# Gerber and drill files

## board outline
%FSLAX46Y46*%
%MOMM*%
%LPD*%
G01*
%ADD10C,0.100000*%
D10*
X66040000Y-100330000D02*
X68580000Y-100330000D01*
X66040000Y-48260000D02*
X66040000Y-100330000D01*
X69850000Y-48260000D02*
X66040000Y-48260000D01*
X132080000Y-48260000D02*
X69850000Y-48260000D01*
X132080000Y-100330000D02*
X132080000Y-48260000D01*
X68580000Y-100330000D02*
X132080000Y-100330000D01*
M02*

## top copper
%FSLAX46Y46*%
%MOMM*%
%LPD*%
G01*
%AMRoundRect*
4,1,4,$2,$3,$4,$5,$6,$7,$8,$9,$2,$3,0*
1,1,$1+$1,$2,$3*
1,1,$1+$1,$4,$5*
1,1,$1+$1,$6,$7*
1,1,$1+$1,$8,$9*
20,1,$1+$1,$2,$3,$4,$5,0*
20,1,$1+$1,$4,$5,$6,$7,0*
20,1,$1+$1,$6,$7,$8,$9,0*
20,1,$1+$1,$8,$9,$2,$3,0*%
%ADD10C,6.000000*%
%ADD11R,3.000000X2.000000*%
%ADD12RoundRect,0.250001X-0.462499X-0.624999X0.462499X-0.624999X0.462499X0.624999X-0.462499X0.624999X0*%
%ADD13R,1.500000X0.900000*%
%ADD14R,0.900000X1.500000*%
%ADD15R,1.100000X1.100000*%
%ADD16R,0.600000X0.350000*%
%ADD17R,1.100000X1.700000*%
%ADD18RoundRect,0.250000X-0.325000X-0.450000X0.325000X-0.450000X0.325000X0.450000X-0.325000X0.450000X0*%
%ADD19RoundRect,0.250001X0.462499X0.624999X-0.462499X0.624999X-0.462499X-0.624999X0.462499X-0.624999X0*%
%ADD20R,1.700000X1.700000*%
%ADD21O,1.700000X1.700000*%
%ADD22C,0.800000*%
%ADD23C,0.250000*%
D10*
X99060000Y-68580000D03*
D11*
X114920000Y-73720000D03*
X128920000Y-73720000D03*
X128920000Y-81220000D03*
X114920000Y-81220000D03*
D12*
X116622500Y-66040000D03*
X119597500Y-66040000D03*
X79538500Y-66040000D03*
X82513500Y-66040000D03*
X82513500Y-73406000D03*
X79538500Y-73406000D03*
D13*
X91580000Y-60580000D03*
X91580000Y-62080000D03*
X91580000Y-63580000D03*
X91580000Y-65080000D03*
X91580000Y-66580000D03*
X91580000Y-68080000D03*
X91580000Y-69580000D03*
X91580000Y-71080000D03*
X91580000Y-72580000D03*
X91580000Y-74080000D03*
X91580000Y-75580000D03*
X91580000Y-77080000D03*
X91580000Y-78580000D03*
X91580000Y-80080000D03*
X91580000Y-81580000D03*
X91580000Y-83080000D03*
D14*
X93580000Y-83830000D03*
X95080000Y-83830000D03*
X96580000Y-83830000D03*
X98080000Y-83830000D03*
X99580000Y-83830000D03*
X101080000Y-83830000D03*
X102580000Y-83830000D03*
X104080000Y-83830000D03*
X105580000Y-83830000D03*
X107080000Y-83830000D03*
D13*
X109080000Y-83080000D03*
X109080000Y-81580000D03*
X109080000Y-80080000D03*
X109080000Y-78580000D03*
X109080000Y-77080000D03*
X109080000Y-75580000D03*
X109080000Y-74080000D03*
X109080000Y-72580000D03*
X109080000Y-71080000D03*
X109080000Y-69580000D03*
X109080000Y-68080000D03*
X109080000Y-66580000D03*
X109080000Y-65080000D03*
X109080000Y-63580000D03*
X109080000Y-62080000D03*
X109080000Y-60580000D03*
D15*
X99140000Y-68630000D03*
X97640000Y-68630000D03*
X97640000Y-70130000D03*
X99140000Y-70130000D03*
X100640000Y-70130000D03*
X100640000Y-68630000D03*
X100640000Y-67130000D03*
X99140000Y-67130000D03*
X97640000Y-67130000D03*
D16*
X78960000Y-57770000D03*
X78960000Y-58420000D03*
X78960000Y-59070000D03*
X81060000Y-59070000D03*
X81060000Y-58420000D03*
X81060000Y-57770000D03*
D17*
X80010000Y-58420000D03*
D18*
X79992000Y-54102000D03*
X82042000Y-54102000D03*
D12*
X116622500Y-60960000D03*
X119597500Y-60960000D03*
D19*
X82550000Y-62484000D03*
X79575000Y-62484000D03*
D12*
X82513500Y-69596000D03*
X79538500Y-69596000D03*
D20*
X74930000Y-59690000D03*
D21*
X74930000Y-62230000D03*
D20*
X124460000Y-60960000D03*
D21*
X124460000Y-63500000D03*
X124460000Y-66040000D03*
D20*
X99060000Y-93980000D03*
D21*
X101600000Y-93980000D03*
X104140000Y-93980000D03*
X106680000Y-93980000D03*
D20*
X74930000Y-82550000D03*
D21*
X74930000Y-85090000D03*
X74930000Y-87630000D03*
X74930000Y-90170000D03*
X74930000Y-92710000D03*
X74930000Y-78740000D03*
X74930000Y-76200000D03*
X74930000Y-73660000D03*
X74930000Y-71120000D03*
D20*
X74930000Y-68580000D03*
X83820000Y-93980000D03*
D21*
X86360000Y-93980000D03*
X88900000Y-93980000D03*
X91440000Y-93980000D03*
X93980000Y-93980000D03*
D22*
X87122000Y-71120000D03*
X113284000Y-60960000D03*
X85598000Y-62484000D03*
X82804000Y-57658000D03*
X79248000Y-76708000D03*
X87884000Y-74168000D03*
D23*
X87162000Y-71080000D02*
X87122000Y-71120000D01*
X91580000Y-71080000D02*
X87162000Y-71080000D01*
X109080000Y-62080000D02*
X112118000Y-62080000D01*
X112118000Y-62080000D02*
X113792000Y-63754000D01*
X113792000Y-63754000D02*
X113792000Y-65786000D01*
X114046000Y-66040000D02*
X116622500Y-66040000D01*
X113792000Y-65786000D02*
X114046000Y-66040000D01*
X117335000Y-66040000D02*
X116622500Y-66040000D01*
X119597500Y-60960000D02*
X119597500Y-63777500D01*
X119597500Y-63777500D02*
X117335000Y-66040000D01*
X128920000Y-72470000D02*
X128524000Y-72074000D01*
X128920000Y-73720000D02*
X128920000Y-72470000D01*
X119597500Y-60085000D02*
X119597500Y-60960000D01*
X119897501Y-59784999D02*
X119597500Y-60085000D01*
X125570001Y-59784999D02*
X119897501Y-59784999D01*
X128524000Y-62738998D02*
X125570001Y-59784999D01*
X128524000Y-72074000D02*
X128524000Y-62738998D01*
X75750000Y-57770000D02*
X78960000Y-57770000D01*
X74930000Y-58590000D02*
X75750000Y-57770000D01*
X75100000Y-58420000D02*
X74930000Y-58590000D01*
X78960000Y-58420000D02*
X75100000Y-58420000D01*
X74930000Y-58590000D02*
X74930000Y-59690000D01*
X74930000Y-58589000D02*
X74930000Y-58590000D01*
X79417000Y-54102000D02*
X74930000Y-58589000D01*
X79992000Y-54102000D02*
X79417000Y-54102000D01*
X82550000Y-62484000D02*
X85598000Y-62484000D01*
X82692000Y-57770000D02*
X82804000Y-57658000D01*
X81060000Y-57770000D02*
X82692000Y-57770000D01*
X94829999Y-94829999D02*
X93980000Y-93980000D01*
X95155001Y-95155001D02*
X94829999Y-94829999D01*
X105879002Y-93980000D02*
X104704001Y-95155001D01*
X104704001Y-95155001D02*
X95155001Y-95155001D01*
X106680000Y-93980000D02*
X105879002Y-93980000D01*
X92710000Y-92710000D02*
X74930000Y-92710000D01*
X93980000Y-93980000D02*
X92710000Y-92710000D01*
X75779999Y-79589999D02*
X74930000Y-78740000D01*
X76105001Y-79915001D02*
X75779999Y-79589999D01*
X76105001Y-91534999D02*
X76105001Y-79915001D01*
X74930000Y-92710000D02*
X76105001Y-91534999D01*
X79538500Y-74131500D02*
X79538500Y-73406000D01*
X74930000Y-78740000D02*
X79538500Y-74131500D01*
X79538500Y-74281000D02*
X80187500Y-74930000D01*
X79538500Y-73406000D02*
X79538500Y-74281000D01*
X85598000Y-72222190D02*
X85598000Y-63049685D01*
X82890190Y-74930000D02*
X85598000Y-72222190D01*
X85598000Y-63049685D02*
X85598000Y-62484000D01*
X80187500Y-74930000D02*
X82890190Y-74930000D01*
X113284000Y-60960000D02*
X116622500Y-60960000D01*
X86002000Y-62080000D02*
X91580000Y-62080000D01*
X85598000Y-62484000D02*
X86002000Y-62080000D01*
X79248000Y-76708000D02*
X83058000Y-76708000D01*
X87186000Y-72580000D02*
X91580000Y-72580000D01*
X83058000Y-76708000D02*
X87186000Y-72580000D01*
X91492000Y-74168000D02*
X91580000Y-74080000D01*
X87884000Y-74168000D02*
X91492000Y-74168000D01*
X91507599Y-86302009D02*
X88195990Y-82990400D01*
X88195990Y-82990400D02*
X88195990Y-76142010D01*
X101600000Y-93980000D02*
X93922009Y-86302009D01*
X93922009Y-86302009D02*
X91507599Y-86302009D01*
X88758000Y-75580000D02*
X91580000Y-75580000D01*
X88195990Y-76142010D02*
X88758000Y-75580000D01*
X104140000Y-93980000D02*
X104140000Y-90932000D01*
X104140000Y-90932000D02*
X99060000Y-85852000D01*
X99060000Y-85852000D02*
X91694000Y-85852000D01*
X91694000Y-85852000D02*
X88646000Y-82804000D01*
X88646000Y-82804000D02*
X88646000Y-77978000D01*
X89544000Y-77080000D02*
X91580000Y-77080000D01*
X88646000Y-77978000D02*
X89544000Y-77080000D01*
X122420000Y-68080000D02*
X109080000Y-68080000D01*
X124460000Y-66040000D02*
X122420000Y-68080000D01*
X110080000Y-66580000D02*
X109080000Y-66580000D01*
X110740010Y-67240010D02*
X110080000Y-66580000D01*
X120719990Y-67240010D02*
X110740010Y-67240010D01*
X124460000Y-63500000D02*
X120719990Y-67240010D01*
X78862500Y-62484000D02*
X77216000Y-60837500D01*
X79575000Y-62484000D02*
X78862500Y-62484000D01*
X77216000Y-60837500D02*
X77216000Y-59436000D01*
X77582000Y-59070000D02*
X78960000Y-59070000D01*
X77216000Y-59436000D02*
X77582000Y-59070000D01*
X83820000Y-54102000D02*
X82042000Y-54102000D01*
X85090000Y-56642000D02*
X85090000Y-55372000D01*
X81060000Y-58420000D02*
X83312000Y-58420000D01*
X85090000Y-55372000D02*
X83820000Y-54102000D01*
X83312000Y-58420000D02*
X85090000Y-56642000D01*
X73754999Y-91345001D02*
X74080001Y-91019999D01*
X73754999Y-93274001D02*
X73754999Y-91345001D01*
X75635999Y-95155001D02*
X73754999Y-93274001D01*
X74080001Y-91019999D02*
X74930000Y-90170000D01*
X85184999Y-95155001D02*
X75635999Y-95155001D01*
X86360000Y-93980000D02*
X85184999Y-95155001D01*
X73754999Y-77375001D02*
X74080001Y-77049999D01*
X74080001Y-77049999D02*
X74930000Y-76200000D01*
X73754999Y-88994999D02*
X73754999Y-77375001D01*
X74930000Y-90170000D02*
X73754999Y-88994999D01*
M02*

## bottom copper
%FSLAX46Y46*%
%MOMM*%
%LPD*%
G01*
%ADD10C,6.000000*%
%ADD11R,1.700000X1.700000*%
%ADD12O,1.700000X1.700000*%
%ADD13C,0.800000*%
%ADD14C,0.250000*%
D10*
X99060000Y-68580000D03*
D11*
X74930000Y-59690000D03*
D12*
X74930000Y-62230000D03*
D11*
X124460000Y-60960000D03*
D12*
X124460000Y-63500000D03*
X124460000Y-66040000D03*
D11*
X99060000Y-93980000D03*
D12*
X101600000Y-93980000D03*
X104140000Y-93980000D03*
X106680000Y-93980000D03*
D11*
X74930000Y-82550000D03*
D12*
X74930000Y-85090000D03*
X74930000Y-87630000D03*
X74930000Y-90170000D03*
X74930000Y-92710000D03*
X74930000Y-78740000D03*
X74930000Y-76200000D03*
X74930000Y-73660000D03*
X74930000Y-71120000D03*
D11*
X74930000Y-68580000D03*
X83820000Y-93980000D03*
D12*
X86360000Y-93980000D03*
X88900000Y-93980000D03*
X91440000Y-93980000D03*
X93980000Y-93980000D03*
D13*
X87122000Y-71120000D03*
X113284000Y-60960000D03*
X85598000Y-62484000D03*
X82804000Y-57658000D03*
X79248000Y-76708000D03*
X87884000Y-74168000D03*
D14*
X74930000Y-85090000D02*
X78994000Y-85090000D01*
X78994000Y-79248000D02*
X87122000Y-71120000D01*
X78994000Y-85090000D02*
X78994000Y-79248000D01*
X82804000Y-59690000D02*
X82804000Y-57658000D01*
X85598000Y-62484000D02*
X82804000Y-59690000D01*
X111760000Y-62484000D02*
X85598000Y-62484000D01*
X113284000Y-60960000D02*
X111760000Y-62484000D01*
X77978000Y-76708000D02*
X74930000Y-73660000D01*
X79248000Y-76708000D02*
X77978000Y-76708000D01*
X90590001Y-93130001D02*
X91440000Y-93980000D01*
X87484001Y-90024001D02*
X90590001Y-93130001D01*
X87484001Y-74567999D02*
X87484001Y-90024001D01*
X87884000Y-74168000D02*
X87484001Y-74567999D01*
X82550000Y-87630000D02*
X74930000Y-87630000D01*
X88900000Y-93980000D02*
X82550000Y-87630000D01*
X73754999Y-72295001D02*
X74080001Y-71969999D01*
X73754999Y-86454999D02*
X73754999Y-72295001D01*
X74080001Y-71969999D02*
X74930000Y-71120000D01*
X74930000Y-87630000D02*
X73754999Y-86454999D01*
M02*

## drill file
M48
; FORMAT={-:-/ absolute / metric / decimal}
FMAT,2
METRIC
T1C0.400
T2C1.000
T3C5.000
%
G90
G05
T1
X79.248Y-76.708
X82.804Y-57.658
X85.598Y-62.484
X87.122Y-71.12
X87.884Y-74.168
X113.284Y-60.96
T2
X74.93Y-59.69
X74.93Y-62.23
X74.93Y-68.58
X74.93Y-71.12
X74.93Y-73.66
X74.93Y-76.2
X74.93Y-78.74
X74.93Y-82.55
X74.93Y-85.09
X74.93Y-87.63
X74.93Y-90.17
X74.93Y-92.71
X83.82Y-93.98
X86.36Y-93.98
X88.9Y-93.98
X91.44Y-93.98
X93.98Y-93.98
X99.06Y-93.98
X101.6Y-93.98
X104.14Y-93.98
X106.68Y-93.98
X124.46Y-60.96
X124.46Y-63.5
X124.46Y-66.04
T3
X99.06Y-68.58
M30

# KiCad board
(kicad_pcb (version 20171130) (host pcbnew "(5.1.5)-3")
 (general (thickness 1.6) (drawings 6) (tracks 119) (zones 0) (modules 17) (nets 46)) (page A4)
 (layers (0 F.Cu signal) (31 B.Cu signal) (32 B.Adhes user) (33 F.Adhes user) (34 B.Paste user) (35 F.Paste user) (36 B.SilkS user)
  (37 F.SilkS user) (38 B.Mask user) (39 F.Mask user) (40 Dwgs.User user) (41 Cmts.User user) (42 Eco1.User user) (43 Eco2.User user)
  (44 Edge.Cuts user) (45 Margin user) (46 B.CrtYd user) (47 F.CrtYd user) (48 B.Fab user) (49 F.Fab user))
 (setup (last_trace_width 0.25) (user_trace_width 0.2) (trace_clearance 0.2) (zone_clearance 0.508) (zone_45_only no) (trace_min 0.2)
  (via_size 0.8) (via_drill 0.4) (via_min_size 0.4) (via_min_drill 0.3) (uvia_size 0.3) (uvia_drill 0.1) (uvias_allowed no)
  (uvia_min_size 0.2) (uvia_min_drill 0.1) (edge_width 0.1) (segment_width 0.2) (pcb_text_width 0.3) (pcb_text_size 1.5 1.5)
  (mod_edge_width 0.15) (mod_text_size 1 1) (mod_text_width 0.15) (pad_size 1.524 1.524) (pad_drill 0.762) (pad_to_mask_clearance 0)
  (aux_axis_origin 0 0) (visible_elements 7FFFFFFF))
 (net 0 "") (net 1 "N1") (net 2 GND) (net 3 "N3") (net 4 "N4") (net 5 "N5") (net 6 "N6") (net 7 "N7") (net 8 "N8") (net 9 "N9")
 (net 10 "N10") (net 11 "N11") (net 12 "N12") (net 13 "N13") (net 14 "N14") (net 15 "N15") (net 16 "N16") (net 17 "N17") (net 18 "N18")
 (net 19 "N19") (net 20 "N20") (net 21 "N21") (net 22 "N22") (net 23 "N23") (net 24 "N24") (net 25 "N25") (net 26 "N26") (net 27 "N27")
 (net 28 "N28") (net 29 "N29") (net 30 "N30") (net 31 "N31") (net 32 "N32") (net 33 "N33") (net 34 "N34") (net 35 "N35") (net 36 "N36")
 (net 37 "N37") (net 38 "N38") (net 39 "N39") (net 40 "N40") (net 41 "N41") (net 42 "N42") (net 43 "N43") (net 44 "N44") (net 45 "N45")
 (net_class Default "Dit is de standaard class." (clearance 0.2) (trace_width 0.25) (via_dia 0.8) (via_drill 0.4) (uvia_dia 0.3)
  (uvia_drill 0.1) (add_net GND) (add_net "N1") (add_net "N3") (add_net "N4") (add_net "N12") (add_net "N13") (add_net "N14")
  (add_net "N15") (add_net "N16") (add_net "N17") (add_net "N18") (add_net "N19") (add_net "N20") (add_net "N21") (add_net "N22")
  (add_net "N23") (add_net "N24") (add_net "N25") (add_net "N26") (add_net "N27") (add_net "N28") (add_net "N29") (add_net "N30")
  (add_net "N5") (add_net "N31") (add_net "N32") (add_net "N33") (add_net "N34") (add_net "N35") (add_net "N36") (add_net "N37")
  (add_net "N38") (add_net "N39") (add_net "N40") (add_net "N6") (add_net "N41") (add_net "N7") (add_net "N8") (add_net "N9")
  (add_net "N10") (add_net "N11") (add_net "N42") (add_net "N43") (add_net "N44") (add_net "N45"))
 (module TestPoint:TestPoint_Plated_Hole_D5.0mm (layer F.Cu) (at 99.06 68.58)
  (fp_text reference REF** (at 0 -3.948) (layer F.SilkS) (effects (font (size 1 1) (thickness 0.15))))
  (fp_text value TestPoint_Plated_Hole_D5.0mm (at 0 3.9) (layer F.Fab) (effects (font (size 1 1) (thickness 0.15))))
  (pad 1 thru_hole circle (at 0 0) (size 6 6) (drill 5) (layers *.Cu *.Mask)))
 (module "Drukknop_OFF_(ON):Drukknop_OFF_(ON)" (layer F.Cu) (at 121.92 77.47)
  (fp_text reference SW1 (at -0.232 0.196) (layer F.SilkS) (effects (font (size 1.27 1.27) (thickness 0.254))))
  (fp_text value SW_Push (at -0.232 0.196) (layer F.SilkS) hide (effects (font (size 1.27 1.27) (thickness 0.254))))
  (pad 4 smd rect (at -7 -3.75 90) (size 2 3) (layers F.Cu F.Paste F.Mask))
  (pad 3 smd rect (at 7 -3.75 90) (size 2 3) (layers F.Cu F.Paste F.Mask) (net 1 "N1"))
  (pad 2 smd rect (at 7 3.75 90) (size 2 3) (layers F.Cu F.Paste F.Mask))
  (pad 1 smd rect (at -7 3.75 90) (size 2 3) (layers F.Cu F.Paste F.Mask) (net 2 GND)))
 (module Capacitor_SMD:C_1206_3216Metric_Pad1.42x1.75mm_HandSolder (layer F.Cu) (at 118.11 66.04)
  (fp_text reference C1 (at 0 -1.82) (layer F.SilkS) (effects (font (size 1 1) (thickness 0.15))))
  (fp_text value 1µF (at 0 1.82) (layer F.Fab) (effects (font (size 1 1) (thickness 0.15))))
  (pad 1 smd roundrect (at -1.4875 0) (size 1.425 1.75) (layers F.Cu F.Paste F.Mask) (roundrect_rratio 0.175439) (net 1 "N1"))
  (pad 2 smd roundrect (at 1.4875 0) (size 1.425 1.75) (layers F.Cu F.Paste F.Mask) (roundrect_rratio 0.175439) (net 2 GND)))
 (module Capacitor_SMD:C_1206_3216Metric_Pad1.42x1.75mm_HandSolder (layer F.Cu) (at 81.026 66.04)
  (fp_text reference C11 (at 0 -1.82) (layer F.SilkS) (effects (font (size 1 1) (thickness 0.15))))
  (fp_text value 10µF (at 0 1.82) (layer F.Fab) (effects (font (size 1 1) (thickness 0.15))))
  (pad 1 smd roundrect (at -1.4875 0) (size 1.425 1.75) (layers F.Cu F.Paste F.Mask) (roundrect_rratio 0.175439) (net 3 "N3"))
  (pad 2 smd roundrect (at 1.4875 0) (size 1.425 1.75) (layers F.Cu F.Paste F.Mask) (roundrect_rratio 0.175439) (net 2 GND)))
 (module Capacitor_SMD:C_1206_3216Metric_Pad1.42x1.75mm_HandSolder (layer F.Cu) (at 81.026 73.406)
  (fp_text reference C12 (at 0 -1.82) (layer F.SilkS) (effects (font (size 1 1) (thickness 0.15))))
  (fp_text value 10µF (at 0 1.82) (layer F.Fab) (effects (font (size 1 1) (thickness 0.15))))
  (pad 2 smd roundrect (at 1.4875 0) (size 1.425 1.75) (layers F.Cu F.Paste F.Mask) (roundrect_rratio 0.175439) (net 2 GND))
  (pad 1 smd roundrect (at -1.4875 0) (size 1.425 1.75) (layers F.Cu F.Paste F.Mask) (roundrect_rratio 0.175439) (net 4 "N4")))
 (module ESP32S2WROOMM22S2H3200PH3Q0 (layer F.Cu) (at 100.33 68.58)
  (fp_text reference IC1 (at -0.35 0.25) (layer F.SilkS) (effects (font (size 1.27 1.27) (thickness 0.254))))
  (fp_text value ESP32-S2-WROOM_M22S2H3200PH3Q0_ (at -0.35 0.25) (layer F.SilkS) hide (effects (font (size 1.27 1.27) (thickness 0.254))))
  (pad 1 smd rect (at -8.75 -8 90) (size 0.9 1.5) (layers F.Cu F.Paste F.Mask) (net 2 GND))
  (pad 2 smd rect (at -8.75 -6.5 90) (size 0.9 1.5) (layers F.Cu F.Paste F.Mask) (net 4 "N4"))
  (pad 3 smd rect (at -8.75 -5 90) (size 0.9 1.5) (layers F.Cu F.Paste F.Mask) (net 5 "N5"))
  (pad 4 smd rect (at -8.75 -3.5 90) (size 0.9 1.5) (layers F.Cu F.Paste F.Mask) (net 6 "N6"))
  (pad 5 smd rect (at -8.75 -2 90) (size 0.9 1.5) (layers F.Cu F.Paste F.Mask) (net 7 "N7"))
  (pad 6 smd rect (at -8.75 -0.5 90) (size 0.9 1.5) (layers F.Cu F.Paste F.Mask) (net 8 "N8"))
  (pad 7 smd rect (at -8.75 1 90) (size 0.9 1.5) (layers F.Cu F.Paste F.Mask) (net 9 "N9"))
  (pad 8 smd rect (at -8.75 2.5 90) (size 0.9 1.5) (layers F.Cu F.Paste F.Mask) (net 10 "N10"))
  (pad 9 smd rect (at -8.75 4 90) (size 0.9 1.5) (layers F.Cu F.Paste F.Mask) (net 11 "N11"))
  (pad 10 smd rect (at -8.75 5.5 90) (size 0.9 1.5) (layers F.Cu F.Paste F.Mask) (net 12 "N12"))
  (pad 11 smd rect (at -8.75 7 90) (size 0.9 1.5) (layers F.Cu F.Paste F.Mask) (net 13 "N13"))
  (pad 12 smd rect (at -8.75 8.5 90) (size 0.9 1.5) (layers F.Cu F.Paste F.Mask) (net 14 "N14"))
  (pad 13 smd rect (at -8.75 10 90) (size 0.9 1.5) (layers F.Cu F.Paste F.Mask) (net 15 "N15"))
  (pad 14 smd rect (at -8.75 11.5 90) (size 0.9 1.5) (layers F.Cu F.Paste F.Mask) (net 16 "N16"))
  (pad 15 smd rect (at -8.75 13 90) (size 0.9 1.5) (layers F.Cu F.Paste F.Mask) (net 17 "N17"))
  (pad 16 smd rect (at -8.75 14.5 90) (size 0.9 1.5) (layers F.Cu F.Paste F.Mask) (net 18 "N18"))
  (pad 17 smd rect (at -6.75 15.25) (size 0.9 1.5) (layers F.Cu F.Paste F.Mask) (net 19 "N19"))
  (pad 18 smd rect (at -5.25 15.25) (size 0.9 1.5) (layers F.Cu F.Paste F.Mask) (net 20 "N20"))
  (pad 19 smd rect (at -3.75 15.25) (size 0.9 1.5) (layers F.Cu F.Paste F.Mask) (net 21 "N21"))
  (pad 20 smd rect (at -2.25 15.25) (size 0.9 1.5) (layers F.Cu F.Paste F.Mask) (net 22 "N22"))
  (pad 21 smd rect (at -0.75 15.25) (size 0.9 1.5) (layers F.Cu F.Paste F.Mask) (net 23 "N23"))
  (pad 22 smd rect (at 0.75 15.25) (size 0.9 1.5) (layers F.Cu F.Paste F.Mask) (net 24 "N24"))
  (pad 23 smd rect (at 2.25 15.25) (size 0.9 1.5) (layers F.Cu F.Paste F.Mask) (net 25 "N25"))
  (pad 24 smd rect (at 3.75 15.25) (size 0.9 1.5) (layers F.Cu F.Paste F.Mask) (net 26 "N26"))
  (pad 25 smd rect (at 5.25 15.25) (size 0.9 1.5) (layers F.Cu F.Paste F.Mask) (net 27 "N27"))
  (pad 26 smd rect (at 6.75 15.25) (size 0.9 1.5) (layers F.Cu F.Paste F.Mask) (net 2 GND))
  (pad 27 smd rect (at 8.75 14.5 90) (size 0.9 1.5) (layers F.Cu F.Paste F.Mask) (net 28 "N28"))
  (pad 28 smd rect (at 8.75 13 90) (size 0.9 1.5) (layers F.Cu F.Paste F.Mask) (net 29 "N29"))
  (pad 29 smd rect (at 8.75 11.5 90) (size 0.9 1.5) (layers F.Cu F.Paste F.Mask) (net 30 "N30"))
  (pad 30 smd rect (at 8.75 10 90) (size 0.9 1.5) (layers F.Cu F.Paste F.Mask) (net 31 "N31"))
  (pad 31 smd rect (at 8.75 8.5 90) (size 0.9 1.5) (layers F.Cu F.Paste F.Mask) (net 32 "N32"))
  (pad 32 smd rect (at 8.75 7 90) (size 0.9 1.5) (layers F.Cu F.Paste F.Mask) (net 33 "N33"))
  (pad 33 smd rect (at 8.75 5.5 90) (size 0.9 1.5) (layers F.Cu F.Paste F.Mask) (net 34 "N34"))
  (pad 34 smd rect (at 8.75 4 90) (size 0.9 1.5) (layers F.Cu F.Paste F.Mask) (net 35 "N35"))
  (pad 35 smd rect (at 8.75 2.5 90) (size 0.9 1.5) (layers F.Cu F.Paste F.Mask) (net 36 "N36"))
  (pad 36 smd rect (at 8.75 1 90) (size 0.9 1.5) (layers F.Cu F.Paste F.Mask) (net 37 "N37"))
  (pad 37 smd rect (at 8.75 -0.5 90) (size 0.9 1.5) (layers F.Cu F.Paste F.Mask) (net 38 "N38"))
  (pad 38 smd rect (at 8.75 -2 90) (size 0.9 1.5) (layers F.Cu F.Paste F.Mask) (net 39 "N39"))
  (pad 39 smd rect (at 8.75 -3.5 90) (size 0.9 1.5) (layers F.Cu F.Paste F.Mask) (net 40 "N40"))
  (pad 40 smd rect (at 8.75 -5 90) (size 0.9 1.5) (layers F.Cu F.Paste F.Mask) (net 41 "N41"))
  (pad 41 smd rect (at 8.75 -6.5 90) (size 0.9 1.5) (layers F.Cu F.Paste F.Mask) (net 1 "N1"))
  (pad 42 smd rect (at 8.75 -8 90) (size 0.9 1.5) (layers F.Cu F.Paste F.Mask) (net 2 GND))
  (pad 43 smd rect (at -1.19 0.05) (size 1.1 1.1) (layers F.Cu F.Paste F.Mask) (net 2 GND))
  (pad 44 smd rect (at -2.69 0.05) (size 1.1 1.1) (layers F.Cu F.Paste F.Mask) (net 2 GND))
  (pad 45 smd rect (at -2.69 1.55) (size 1.1 1.1) (layers F.Cu F.Paste F.Mask) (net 2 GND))
  (pad 46 smd rect (at -1.19 1.55) (size 1.1 1.1) (layers F.Cu F.Paste F.Mask) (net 2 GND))
  (pad 47 smd rect (at 0.31 1.55) (size 1.1 1.1) (layers F.Cu F.Paste F.Mask) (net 2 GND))
  (pad 48 smd rect (at 0.31 0.05) (size 1.1 1.1) (layers F.Cu F.Paste F.Mask) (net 2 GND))
  (pad 49 smd rect (at 0.31 -1.45) (size 1.1 1.1) (layers F.Cu F.Paste F.Mask) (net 2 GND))
  (pad 50 smd rect (at -1.19 -1.45) (size 1.1 1.1) (layers F.Cu F.Paste F.Mask) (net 2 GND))
  (pad 51 smd rect (at -2.69 -1.45) (size 1.1 1.1) (layers F.Cu F.Paste F.Mask) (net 2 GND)))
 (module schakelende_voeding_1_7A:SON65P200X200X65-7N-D (layer F.Cu) (at 80.01 58.42)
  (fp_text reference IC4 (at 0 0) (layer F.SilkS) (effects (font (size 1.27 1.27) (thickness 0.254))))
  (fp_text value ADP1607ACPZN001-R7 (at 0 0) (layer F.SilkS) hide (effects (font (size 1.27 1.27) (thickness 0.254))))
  (pad 1 smd rect (at -1.05 -0.65 90) (size 0.35 0.6) (layers F.Cu F.Paste F.Mask) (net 3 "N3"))
  (pad 2 smd rect (at -1.05 0 90) (size 0.35 0.6) (layers F.Cu F.Paste F.Mask) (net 3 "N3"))
  (pad 3 smd rect (at -1.05 0.65 90) (size 0.35 0.6) (layers F.Cu F.Paste F.Mask) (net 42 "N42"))
  (pad 4 smd rect (at 1.05 0.65 90) (size 0.35 0.6) (layers F.Cu F.Paste F.Mask) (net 2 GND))
  (pad 5 smd rect (at 1.05 0 90) (size 0.35 0.6) (layers F.Cu F.Paste F.Mask) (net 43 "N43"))
  (pad 6 smd rect (at 1.05 -0.65 90) (size 0.35 0.6) (layers F.Cu F.Paste F.Mask) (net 4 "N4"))
  (pad 7 smd rect (at 0 0) (size 1.1 1.7) (layers F.Cu F.Paste F.Mask) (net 2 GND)))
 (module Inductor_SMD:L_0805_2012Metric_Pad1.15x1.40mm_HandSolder (layer F.Cu) (at 81.017 54.102)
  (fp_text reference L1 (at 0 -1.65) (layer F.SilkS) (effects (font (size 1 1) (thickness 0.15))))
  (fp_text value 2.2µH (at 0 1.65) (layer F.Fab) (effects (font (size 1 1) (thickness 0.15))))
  (pad 1 smd roundrect (at -1.025 0) (size 1.15 1.4) (layers F.Cu F.Paste F.Mask) (roundrect_rratio 0.217391) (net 3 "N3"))
  (pad 2 smd roundrect (at 1.025 0) (size 1.15 1.4) (layers F.Cu F.Paste F.Mask) (roundrect_rratio 0.217391) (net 43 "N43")))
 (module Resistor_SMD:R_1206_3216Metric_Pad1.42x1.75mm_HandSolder (layer F.Cu) (at 118.11 60.96)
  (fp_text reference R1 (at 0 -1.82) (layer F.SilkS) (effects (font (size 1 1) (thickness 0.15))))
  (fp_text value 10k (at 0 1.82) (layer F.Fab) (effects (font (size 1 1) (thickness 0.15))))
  (pad 1 smd roundrect (at -1.4875 0) (size 1.425 1.75) (layers F.Cu F.Paste F.Mask) (roundrect_rratio 0.175439) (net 4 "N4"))
  (pad 2 smd roundrect (at 1.4875 0) (size 1.425 1.75) (layers F.Cu F.Paste F.Mask) (roundrect_rratio 0.175439) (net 1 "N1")))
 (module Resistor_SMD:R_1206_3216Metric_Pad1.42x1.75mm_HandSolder (layer F.Cu) (at 81.0625 62.484 180)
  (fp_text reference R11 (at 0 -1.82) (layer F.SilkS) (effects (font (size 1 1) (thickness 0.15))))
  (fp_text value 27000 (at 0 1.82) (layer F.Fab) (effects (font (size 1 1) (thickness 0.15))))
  (pad 1 smd roundrect (at -1.4875 0 180) (size 1.425 1.75) (layers F.Cu F.Paste F.Mask) (roundrect_rratio 0.175439) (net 4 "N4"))
  (pad 2 smd roundrect (at 1.4875 0 180) (size 1.425 1.75) (layers F.Cu F.Paste F.Mask) (roundrect_rratio 0.175439) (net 42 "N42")))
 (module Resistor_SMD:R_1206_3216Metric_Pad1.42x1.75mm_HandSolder (layer F.Cu) (at 81.026 69.596)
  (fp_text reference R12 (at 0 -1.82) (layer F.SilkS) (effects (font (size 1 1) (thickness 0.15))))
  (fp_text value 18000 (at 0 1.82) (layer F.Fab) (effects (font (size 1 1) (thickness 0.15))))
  (pad 2 smd roundrect (at 1.4875 0) (size 1.425 1.75) (layers F.Cu F.Paste F.Mask) (roundrect_rratio 0.175439) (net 2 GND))
  (pad 1 smd roundrect (at -1.4875 0) (size 1.425 1.75) (layers F.Cu F.Paste F.Mask) (roundrect_rratio 0.175439) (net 42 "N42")))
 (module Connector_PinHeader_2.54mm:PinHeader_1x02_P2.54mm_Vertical (layer F.Cu) (at 74.93 59.69)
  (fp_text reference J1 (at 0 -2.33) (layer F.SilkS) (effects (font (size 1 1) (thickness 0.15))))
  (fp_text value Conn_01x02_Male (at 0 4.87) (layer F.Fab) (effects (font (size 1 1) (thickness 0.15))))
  (pad 1 thru_hole rect (at 0 0) (size 1.7 1.7) (drill 1) (layers *.Cu *.Mask) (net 3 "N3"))
  (pad 2 thru_hole oval (at 0 2.54) (size 1.7 1.7) (drill 1) (layers *.Cu *.Mask) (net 2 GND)))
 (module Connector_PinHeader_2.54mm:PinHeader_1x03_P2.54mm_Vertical (layer F.Cu) (at 124.46 60.96)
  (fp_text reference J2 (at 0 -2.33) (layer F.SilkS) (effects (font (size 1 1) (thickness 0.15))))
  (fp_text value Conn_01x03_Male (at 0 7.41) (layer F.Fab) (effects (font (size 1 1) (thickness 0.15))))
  (pad 1 thru_hole rect (at 0 0) (size 1.7 1.7) (drill 1) (layers *.Cu *.Mask) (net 2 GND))
  (pad 2 thru_hole oval (at 0 2.54) (size 1.7 1.7) (drill 1) (layers *.Cu *.Mask) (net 39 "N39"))
  (pad 3 thru_hole oval (at 0 5.08) (size 1.7 1.7) (drill 1) (layers *.Cu *.Mask) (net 38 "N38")))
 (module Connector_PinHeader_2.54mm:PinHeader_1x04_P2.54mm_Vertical (layer F.Cu) (at 99.06 93.98 90)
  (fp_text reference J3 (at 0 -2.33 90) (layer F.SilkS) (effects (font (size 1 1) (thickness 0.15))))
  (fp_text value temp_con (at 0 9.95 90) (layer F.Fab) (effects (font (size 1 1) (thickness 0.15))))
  (pad 1 thru_hole rect (at 0 0 90) (size 1.7 1.7) (drill 1) (layers *.Cu *.Mask) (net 2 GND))
  (pad 2 thru_hole oval (at 0 2.54 90) (size 1.7 1.7) (drill 1) (layers *.Cu *.Mask) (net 13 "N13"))
  (pad 3 thru_hole oval (at 0 5.08 90) (size 1.7 1.7) (drill 1) (layers *.Cu *.Mask) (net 14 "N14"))
  (pad 4 thru_hole oval (at 0 7.62 90) (size 1.7 1.7) (drill 1) (layers *.Cu *.Mask) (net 4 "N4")))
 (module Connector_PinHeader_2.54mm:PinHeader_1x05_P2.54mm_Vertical (layer F.Cu) (at 74.93 82.55)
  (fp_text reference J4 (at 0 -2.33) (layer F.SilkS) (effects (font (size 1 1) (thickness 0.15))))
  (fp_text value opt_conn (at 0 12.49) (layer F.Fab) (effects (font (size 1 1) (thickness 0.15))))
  (pad 1 thru_hole rect (at 0 0) (size 1.7 1.7) (drill 1) (layers *.Cu *.Mask) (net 2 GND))
  (pad 2 thru_hole oval (at 0 2.54) (size 1.7 1.7) (drill 1) (layers *.Cu *.Mask) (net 10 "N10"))
  (pad 3 thru_hole oval (at 0 5.08) (size 1.7 1.7) (drill 1) (layers *.Cu *.Mask) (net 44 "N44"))
  (pad 4 thru_hole oval (at 0 7.62) (size 1.7 1.7) (drill 1) (layers *.Cu *.Mask) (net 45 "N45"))
  (pad 5 thru_hole oval (at 0 10.16) (size 1.7 1.7) (drill 1) (layers *.Cu *.Mask) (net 4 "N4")))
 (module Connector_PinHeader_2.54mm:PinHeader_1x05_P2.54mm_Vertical (layer F.Cu) (at 74.93 68.58)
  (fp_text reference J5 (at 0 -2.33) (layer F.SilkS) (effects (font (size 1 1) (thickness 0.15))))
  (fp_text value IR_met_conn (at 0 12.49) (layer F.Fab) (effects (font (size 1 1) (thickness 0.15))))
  (pad 5 thru_hole oval (at 0 10.16) (size 1.7 1.7) (drill 1) (layers *.Cu *.Mask) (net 4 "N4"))
  (pad 4 thru_hole oval (at 0 7.62) (size 1.7 1.7) (drill 1) (layers *.Cu *.Mask) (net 45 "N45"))
  (pad 3 thru_hole oval (at 0 5.08) (size 1.7 1.7) (drill 1) (layers *.Cu *.Mask) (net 11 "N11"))
  (pad 2 thru_hole oval (at 0 2.54) (size 1.7 1.7) (drill 1) (layers *.Cu *.Mask) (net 44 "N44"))
  (pad 1 thru_hole rect (at 0 0) (size 1.7 1.7) (drill 1) (layers *.Cu *.Mask) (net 2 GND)))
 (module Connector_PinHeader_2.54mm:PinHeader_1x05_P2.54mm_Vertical (layer F.Cu) (at 83.82 93.98 90)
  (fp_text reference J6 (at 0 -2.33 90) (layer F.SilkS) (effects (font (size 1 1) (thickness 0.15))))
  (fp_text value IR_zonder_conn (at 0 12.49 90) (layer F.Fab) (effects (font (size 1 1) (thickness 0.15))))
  (pad 1 thru_hole rect (at 0 0 90) (size 1.7 1.7) (drill 1) (layers *.Cu *.Mask) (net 2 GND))
  (pad 2 thru_hole oval (at 0 2.54 90) (size 1.7 1.7) (drill 1) (layers *.Cu *.Mask) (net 45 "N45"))
  (pad 3 thru_hole oval (at 0 5.08 90) (size 1.7 1.7) (drill 1) (layers *.Cu *.Mask) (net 44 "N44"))
  (pad 4 thru_hole oval (at 0 7.62 90) (size 1.7 1.7) (drill 1) (layers *.Cu *.Mask) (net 12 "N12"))
  (pad 5 thru_hole oval (at 0 10.16 90) (size 1.7 1.7) (drill 1) (layers *.Cu *.Mask) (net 4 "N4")))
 (gr_line (start 66.04 100.33) (end 68.58 100.33) (layer Edge.Cuts) (width 0.1))
 (gr_line (start 66.04 48.26) (end 66.04 100.33) (layer Edge.Cuts) (width 0.1))
 (gr_line (start 69.85 48.26) (end 66.04 48.26) (layer Edge.Cuts) (width 0.1))
 (gr_line (start 132.08 48.26) (end 69.85 48.26) (layer Edge.Cuts) (width 0.1))
 (gr_line (start 132.08 100.33) (end 132.08 48.26) (layer Edge.Cuts) (width 0.1))
 (gr_line (start 68.58 100.33) (end 132.08 100.33) (layer Edge.Cuts) (width 0.1))
 (via (at 87.122 71.12) (size 0.8) (drill 0.4) (layers F.Cu B.Cu) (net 10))
 (segment (start 87.162 71.08) (end 87.122 71.12) (width 0.25) (layer F.Cu) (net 10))
 (segment (start 91.58 71.08) (end 87.162 71.08) (width 0.25) (layer F.Cu) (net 10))
 (segment (start 74.93 85.09) (end 78.994 85.09) (width 0.25) (layer B.Cu) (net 10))
 (segment (start 78.994 79.248) (end 87.122 71.12) (width 0.25) (layer B.Cu) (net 10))
 (segment (start 78.994 85.09) (end 78.994 79.248) (width 0.25) (layer B.Cu) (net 10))
 (segment (start 109.08 62.08) (end 112.118 62.08) (width 0.25) (layer F.Cu) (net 1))
 (segment (start 112.118 62.08) (end 113.792 63.754) (width 0.25) (layer F.Cu) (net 1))
 (segment (start 113.792 63.754) (end 113.792 65.786) (width 0.25) (layer F.Cu) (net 1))
 (segment (start 114.046 66.04) (end 116.6225 66.04) (width 0.25) (layer F.Cu) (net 1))
 (segment (start 113.792 65.786) (end 114.046 66.04) (width 0.25) (layer F.Cu) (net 1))
 (segment (start 117.335 66.04) (end 116.6225 66.04) (width 0.25) (layer F.Cu) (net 1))
 (segment (start 119.5975 60.96) (end 119.5975 63.7775) (width 0.25) (layer F.Cu) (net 1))
 (segment (start 119.5975 63.7775) (end 117.335 66.04) (width 0.25) (layer F.Cu) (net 1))
 (segment (start 128.92 72.47) (end 128.524 72.074) (width 0.25) (layer F.Cu) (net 1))
 (segment (start 128.92 73.72) (end 128.92 72.47) (width 0.25) (layer F.Cu) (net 1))
 (segment (start 119.5975 60.085) (end 119.5975 60.96) (width 0.25) (layer F.Cu) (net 1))
 (segment (start 119.897501 59.784999) (end 119.5975 60.085) (width 0.25) (layer F.Cu) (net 1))
 (segment (start 125.570001 59.784999) (end 119.897501 59.784999) (width 0.25) (layer F.Cu) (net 1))
 (segment (start 128.524 62.738998) (end 125.570001 59.784999) (width 0.25) (layer F.Cu) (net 1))
 (segment (start 128.524 72.074) (end 128.524 62.738998) (width 0.25) (layer F.Cu) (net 1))
 (segment (start 75.75 57.77) (end 78.96 57.77) (width 0.25) (layer F.Cu) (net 3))
 (segment (start 74.93 58.59) (end 75.75 57.77) (width 0.25) (layer F.Cu) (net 3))
 (segment (start 75.1 58.42) (end 74.93 58.59) (width 0.25) (layer F.Cu) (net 3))
 (segment (start 78.96 58.42) (end 75.1 58.42) (width 0.25) (layer F.Cu) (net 3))
 (segment (start 74.93 58.59) (end 74.93 59.69) (width 0.25) (layer F.Cu) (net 3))
 (segment (start 74.93 58.589) (end 74.93 58.59) (width 0.25) (layer F.Cu) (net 3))
 (segment (start 79.417 54.102) (end 74.93 58.589) (width 0.25) (layer F.Cu) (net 3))
 (segment (start 79.992 54.102) (end 79.417 54.102) (width 0.25) (layer F.Cu) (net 3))
 (via (at 113.284 60.96) (size 0.8) (drill 0.4) (layers F.Cu B.Cu) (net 4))
 (via (at 85.598 62.484) (size 0.8) (drill 0.4) (layers F.Cu B.Cu) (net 4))
 (via (at 82.804 57.658) (size 0.8) (drill 0.4) (layers F.Cu B.Cu) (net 4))
 (segment (start 82.55 62.484) (end 85.598 62.484) (width 0.25) (layer F.Cu) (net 4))
 (segment (start 82.692 57.77) (end 82.804 57.658) (width 0.25) (layer F.Cu) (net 4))
 (segment (start 81.06 57.77) (end 82.692 57.77) (width 0.25) (layer F.Cu) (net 4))
 (segment (start 82.804 59.69) (end 82.804 57.658) (width 0.25) (layer B.Cu) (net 4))
 (segment (start 85.598 62.484) (end 82.804 59.69) (width 0.25) (layer B.Cu) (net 4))
 (segment (start 94.829999 94.829999) (end 93.98 93.98) (width 0.25) (layer F.Cu) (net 4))
 (segment (start 95.155001 95.155001) (end 94.829999 94.829999) (width 0.25) (layer F.Cu) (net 4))
 (segment (start 105.879002 93.98) (end 104.704001 95.155001) (width 0.25) (layer F.Cu) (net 4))
 (segment (start 104.704001 95.155001) (end 95.155001 95.155001) (width 0.25) (layer F.Cu) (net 4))
 (segment (start 106.68 93.98) (end 105.879002 93.98) (width 0.25) (layer F.Cu) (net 4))
 (segment (start 92.71 92.71) (end 74.93 92.71) (width 0.25) (layer F.Cu) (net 4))
 (segment (start 93.98 93.98) (end 92.71 92.71) (width 0.25) (layer F.Cu) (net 4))
 (segment (start 75.779999 79.589999) (end 74.93 78.74) (width 0.25) (layer F.Cu) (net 4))
 (segment (start 76.105001 79.915001) (end 75.779999 79.589999) (width 0.25) (layer F.Cu) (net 4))
 (segment (start 76.105001 91.534999) (end 76.105001 79.915001) (width 0.25) (layer F.Cu) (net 4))
 (segment (start 74.93 92.71) (end 76.105001 91.534999) (width 0.25) (layer F.Cu) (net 4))
 (segment (start 79.5385 74.1315) (end 79.5385 73.406) (width 0.25) (layer F.Cu) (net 4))
 (segment (start 74.93 78.74) (end 79.5385 74.1315) (width 0.25) (layer F.Cu) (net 4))
 (segment (start 79.5385 74.281) (end 80.1875 74.93) (width 0.25) (layer F.Cu) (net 4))
 (segment (start 79.5385 73.406) (end 79.5385 74.281) (width 0.25) (layer F.Cu) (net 4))
 (segment (start 85.598 72.22219) (end 85.598 63.049685) (width 0.25) (layer F.Cu) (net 4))
 (segment (start 82.89019 74.93) (end 85.598 72.22219) (width 0.25) (layer F.Cu) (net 4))
 (segment (start 85.598 63.049685) (end 85.598 62.484) (width 0.25) (layer F.Cu) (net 4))
 (segment (start 80.1875 74.93) (end 82.89019 74.93) (width 0.25) (layer F.Cu) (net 4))
 (segment (start 113.284 60.96) (end 116.6225 60.96) (width 0.25) (layer F.Cu) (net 4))
 (segment (start 111.76 62.484) (end 85.598 62.484) (width 0.25) (layer B.Cu) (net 4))
 (segment (start 113.284 60.96) (end 111.76 62.484) (width 0.25) (layer B.Cu) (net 4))
 (segment (start 86.002 62.08) (end 91.58 62.08) (width 0.25) (layer F.Cu) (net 4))
 (segment (start 85.598 62.484) (end 86.002 62.08) (width 0.25) (layer F.Cu) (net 4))
 (via (at 79.248 76.708) (size 0.8) (drill 0.4) (layers F.Cu B.Cu) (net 11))
 (segment (start 77.978 76.708) (end 74.93 73.66) (width 0.25) (layer B.Cu) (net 11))
 (segment (start 79.248 76.708) (end 77.978 76.708) (width 0.25) (layer B.Cu) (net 11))
 (segment (start 79.248 76.708) (end 83.058 76.708) (width 0.25) (layer F.Cu) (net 11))
 (segment (start 87.186 72.58) (end 91.58 72.58) (width 0.25) (layer F.Cu) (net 11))
 (segment (start 83.058 76.708) (end 87.186 72.58) (width 0.25) (layer F.Cu) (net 11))
 (via (at 87.884 74.168) (size 0.8) (drill 0.4) (layers F.Cu B.Cu) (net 12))
 (segment (start 91.492 74.168) (end 91.58 74.08) (width 0.25) (layer F.Cu) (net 12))
 (segment (start 87.884 74.168) (end 91.492 74.168) (width 0.25) (layer F.Cu) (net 12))
 (segment (start 90.590001 93.130001) (end 91.44 93.98) (width 0.25) (layer B.Cu) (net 12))
 (segment (start 87.484001 90.024001) (end 90.590001 93.130001) (width 0.25) (layer B.Cu) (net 12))
 (segment (start 87.484001 74.567999) (end 87.484001 90.024001) (width 0.25) (layer B.Cu) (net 12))
 (segment (start 87.884 74.168) (end 87.484001 74.567999) (width 0.25) (layer B.Cu) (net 12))
 (segment (start 91.507599 86.302009) (end 88.19599 82.9904) (width 0.25) (layer F.Cu) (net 13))
 (segment (start 88.19599 82.9904) (end 88.19599 76.14201) (width 0.25) (layer F.Cu) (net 13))
 (segment (start 101.6 93.98) (end 93.922009 86.302009) (width 0.25) (layer F.Cu) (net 13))
 (segment (start 93.922009 86.302009) (end 91.507599 86.302009) (width 0.25) (layer F.Cu) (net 13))
 (segment (start 88.758 75.58) (end 91.58 75.58) (width 0.25) (layer F.Cu) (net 13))
 (segment (start 88.19599 76.14201) (end 88.758 75.58) (width 0.25) (layer F.Cu) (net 13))
 (segment (start 104.14 93.98) (end 104.14 90.932) (width 0.25) (layer F.Cu) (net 14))
 (segment (start 104.14 90.932) (end 99.06 85.852) (width 0.25) (layer F.Cu) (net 14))
 (segment (start 99.06 85.852) (end 91.694 85.852) (width 0.25) (layer F.Cu) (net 14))
 (segment (start 91.694 85.852) (end 88.646 82.804) (width 0.25) (layer F.Cu) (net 14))
 (segment (start 88.646 82.804) (end 88.646 77.978) (width 0.25) (layer F.Cu) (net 14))
 (segment (start 89.544 77.08) (end 91.58 77.08) (width 0.25) (layer F.Cu) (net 14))
 (segment (start 88.646 77.978) (end 89.544 77.08) (width 0.25) (layer F.Cu) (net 14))
 (segment (start 122.42 68.08) (end 109.08 68.08) (width 0.25) (layer F.Cu) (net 38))
 (segment (start 124.46 66.04) (end 122.42 68.08) (width 0.25) (layer F.Cu) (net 38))
 (segment (start 110.08 66.58) (end 109.08 66.58) (width 0.25) (layer F.Cu) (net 39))
 (segment (start 110.74001 67.24001) (end 110.08 66.58) (width 0.25) (layer F.Cu) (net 39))
 (segment (start 120.71999 67.24001) (end 110.74001 67.24001) (width 0.25) (layer F.Cu) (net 39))
 (segment (start 124.46 63.5) (end 120.71999 67.24001) (width 0.25) (layer F.Cu) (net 39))
 (segment (start 78.8625 62.484) (end 77.216 60.8375) (width 0.25) (layer F.Cu) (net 42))
 (segment (start 79.575 62.484) (end 78.8625 62.484) (width 0.25) (layer F.Cu) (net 42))
 (segment (start 77.216 60.8375) (end 77.216 59.436) (width 0.25) (layer F.Cu) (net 42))
 (segment (start 77.582 59.07) (end 78.96 59.07) (width 0.25) (layer F.Cu) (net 42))
 (segment (start 77.216 59.436) (end 77.582 59.07) (width 0.25) (layer F.Cu) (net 42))
 (segment (start 83.82 54.102) (end 82.042 54.102) (width 0.25) (layer F.Cu) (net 43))
 (segment (start 85.09 56.642) (end 85.09 55.372) (width 0.25) (layer F.Cu) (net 43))
 (segment (start 81.06 58.42) (end 83.312 58.42) (width 0.25) (layer F.Cu) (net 43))
 (segment (start 85.09 55.372) (end 83.82 54.102) (width 0.25) (layer F.Cu) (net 43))
 (segment (start 83.312 58.42) (end 85.09 56.642) (width 0.25) (layer F.Cu) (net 43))
 (segment (start 82.55 87.63) (end 74.93 87.63) (width 0.25) (layer B.Cu) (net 44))
 (segment (start 88.9 93.98) (end 82.55 87.63) (width 0.25) (layer B.Cu) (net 44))
 (segment (start 73.754999 72.295001) (end 74.080001 71.969999) (width 0.25) (layer B.Cu) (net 44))
 (segment (start 73.754999 86.454999) (end 73.754999 72.295001) (width 0.25) (layer B.Cu) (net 44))
 (segment (start 74.080001 71.969999) (end 74.93 71.12) (width 0.25) (layer B.Cu) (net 44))
 (segment (start 74.93 87.63) (end 73.754999 86.454999) (width 0.25) (layer B.Cu) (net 44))
 (segment (start 73.754999 91.345001) (end 74.080001 91.019999) (width 0.25) (layer F.Cu) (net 45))
 (segment (start 73.754999 93.274001) (end 73.754999 91.345001) (width 0.25) (layer F.Cu) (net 45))
 (segment (start 75.635999 95.155001) (end 73.754999 93.274001) (width 0.25) (layer F.Cu) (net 45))
 (segment (start 74.080001 91.019999) (end 74.93 90.17) (width 0.25) (layer F.Cu) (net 45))
 (segment (start 85.184999 95.155001) (end 75.635999 95.155001) (width 0.25) (layer F.Cu) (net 45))
 (segment (start 86.36 93.98) (end 85.184999 95.155001) (width 0.25) (layer F.Cu) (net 45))
 (segment (start 73.754999 77.375001) (end 74.080001 77.049999) (width 0.25) (layer F.Cu) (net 45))
 (segment (start 74.080001 77.049999) (end 74.93 76.2) (width 0.25) (layer F.Cu) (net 45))
 (segment (start 73.754999 88.994999) (end 73.754999 77.375001) (width 0.25) (layer F.Cu) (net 45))
 (segment (start 74.93 90.17) (end 73.754999 88.994999) (width 0.25) (layer F.Cu) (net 45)))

